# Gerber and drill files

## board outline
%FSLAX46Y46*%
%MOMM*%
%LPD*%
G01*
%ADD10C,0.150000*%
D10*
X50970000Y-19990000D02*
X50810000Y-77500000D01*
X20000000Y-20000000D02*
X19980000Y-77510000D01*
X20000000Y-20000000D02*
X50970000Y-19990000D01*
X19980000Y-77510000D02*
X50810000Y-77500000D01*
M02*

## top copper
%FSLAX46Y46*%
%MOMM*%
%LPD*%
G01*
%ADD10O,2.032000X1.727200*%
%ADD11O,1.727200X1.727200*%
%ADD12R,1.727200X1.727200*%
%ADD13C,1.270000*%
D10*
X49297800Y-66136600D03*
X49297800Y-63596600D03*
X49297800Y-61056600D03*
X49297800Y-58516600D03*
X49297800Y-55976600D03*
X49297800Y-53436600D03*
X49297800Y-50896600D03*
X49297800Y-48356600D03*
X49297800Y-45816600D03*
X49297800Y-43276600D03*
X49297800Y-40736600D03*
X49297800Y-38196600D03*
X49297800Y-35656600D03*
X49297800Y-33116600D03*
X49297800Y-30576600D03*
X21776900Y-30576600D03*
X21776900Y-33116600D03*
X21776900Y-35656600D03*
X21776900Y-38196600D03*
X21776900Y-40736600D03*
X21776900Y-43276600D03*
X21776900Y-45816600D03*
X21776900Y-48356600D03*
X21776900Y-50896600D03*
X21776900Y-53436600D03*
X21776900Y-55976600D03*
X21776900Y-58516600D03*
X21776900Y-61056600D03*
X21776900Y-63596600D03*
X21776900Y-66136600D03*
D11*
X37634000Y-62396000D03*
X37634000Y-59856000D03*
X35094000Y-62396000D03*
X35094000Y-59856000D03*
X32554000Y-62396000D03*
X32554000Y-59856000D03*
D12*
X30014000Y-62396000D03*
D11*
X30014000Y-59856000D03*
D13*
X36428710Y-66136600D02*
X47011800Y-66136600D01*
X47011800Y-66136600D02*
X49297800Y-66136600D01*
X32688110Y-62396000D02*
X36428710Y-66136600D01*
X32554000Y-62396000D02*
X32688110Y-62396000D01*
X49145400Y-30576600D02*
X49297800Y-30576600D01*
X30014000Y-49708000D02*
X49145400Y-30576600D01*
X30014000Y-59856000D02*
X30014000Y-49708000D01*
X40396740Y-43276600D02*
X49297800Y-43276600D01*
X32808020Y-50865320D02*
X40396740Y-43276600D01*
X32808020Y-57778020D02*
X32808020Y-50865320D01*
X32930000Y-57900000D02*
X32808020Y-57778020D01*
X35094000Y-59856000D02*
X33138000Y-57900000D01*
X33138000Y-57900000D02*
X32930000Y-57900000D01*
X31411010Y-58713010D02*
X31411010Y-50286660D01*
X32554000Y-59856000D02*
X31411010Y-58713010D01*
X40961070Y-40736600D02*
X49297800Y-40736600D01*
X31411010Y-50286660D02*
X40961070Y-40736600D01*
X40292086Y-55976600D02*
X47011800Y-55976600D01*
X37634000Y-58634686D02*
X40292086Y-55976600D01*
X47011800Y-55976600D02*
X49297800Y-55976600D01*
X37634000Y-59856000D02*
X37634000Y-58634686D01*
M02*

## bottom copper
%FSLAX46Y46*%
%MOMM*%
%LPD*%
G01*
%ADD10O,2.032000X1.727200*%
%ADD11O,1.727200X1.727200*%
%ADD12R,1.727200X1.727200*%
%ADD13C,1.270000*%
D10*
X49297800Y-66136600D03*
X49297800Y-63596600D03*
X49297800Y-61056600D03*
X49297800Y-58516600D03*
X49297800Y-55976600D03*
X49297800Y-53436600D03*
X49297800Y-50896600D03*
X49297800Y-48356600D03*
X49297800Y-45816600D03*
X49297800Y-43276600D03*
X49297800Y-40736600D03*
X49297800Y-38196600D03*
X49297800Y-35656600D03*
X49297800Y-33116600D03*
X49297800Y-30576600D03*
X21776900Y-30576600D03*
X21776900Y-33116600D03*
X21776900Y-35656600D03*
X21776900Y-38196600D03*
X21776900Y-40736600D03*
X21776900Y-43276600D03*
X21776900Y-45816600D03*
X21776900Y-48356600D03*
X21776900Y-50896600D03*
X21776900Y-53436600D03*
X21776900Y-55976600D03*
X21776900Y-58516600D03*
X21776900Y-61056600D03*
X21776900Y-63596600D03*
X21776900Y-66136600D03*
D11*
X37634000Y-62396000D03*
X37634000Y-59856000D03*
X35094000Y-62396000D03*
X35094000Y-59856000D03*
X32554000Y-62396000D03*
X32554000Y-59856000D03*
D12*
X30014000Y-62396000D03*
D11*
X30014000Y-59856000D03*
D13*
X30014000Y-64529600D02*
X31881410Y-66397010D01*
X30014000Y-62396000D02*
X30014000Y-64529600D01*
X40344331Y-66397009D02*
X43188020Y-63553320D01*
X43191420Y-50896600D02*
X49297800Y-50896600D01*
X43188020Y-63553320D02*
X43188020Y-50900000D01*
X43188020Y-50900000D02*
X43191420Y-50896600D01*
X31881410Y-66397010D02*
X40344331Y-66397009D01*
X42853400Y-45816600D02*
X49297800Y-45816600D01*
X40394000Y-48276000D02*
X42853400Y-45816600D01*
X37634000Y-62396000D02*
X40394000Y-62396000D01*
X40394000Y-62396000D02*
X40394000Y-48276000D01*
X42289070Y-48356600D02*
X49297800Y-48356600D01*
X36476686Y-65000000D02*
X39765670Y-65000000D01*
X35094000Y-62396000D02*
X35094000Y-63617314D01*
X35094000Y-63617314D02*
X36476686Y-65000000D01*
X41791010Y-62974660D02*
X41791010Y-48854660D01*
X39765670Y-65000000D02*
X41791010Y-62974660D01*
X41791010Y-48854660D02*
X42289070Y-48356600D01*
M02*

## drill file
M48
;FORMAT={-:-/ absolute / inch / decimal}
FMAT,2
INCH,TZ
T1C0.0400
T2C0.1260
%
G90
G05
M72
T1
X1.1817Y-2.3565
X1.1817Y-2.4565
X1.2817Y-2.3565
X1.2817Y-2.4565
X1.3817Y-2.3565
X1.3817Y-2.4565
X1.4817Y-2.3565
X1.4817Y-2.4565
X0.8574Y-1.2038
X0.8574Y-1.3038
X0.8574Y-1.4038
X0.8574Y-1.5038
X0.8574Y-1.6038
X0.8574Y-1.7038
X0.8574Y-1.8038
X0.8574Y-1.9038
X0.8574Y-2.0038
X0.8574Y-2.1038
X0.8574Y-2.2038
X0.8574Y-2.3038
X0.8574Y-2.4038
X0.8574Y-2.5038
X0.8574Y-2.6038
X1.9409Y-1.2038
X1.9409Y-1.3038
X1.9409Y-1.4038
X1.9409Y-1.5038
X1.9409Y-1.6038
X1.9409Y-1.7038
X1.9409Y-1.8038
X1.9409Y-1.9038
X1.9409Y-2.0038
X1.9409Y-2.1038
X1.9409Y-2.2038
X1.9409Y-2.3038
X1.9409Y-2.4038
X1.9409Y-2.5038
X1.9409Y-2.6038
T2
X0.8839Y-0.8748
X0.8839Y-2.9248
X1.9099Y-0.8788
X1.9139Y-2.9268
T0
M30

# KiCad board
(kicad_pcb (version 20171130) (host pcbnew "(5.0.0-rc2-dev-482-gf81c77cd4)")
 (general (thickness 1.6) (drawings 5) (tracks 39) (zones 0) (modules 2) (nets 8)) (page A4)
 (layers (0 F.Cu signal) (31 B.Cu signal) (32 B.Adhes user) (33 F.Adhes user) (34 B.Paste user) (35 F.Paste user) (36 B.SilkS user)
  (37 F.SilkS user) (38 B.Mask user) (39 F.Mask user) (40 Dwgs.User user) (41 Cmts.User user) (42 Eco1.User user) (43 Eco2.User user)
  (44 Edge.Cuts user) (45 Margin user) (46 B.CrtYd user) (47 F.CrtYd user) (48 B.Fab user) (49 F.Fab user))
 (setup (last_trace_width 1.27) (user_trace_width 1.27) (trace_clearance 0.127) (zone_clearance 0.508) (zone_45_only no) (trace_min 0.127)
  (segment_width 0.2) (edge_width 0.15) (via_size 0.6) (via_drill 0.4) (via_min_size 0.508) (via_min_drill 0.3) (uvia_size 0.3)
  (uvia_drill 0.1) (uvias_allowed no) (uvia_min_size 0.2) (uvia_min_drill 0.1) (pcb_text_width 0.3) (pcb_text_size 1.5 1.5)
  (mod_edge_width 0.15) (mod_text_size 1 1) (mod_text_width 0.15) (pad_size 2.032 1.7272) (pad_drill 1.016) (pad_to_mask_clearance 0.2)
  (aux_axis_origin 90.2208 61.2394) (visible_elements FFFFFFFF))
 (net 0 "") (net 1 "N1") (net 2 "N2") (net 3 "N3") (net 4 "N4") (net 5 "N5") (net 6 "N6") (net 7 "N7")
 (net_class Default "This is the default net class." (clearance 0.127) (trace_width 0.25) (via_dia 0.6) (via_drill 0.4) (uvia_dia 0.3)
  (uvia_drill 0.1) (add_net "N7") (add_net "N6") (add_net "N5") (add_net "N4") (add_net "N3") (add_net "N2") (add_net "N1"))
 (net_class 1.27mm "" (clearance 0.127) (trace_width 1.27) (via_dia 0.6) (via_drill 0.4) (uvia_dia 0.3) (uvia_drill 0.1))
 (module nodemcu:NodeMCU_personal (layer F.Cu) (at 20.5704 20.2896)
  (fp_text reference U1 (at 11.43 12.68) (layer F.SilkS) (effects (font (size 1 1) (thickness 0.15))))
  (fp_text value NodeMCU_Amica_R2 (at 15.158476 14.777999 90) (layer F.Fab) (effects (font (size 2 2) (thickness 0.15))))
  (pad "" np_thru_hole circle (at 27.94 2.032) (size 3.2 3.2) (drill 3.2) (layers *.Cu *.Mask))
  (pad 30 thru_hole oval (at 28.7274 45.847) (size 2.032 1.7272) (drill 1.016) (layers *.Cu *.Mask F.SilkS) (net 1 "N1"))
  (pad 29 thru_hole oval (at 28.7274 43.307) (size 2.032 1.7272) (drill 1.016) (layers *.Cu *.Mask F.SilkS))
  (pad 28 thru_hole oval (at 28.7274 40.767) (size 2.032 1.7272) (drill 1.016) (layers *.Cu *.Mask F.SilkS))
  (pad 27 thru_hole oval (at 28.7274 38.227) (size 2.032 1.7272) (drill 1.016) (layers *.Cu *.Mask F.SilkS))
  (pad 26 thru_hole oval (at 28.7274 35.687) (size 2.032 1.7272) (drill 1.016) (layers *.Cu *.Mask F.SilkS))
  (pad 25 thru_hole oval (at 28.7274 33.147) (size 2.032 1.7272) (drill 1.016) (layers *.Cu *.Mask F.SilkS))
  (pad 24 thru_hole oval (at 28.7274 30.607) (size 2.032 1.7272) (drill 1.016) (layers *.Cu *.Mask F.SilkS) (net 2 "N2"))
  (pad 23 thru_hole oval (at 28.7274 28.067) (size 2.032 1.7272) (drill 1.016) (layers *.Cu *.Mask F.SilkS) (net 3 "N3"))
  (pad 22 thru_hole oval (at 28.7274 25.527) (size 2.032 1.7272) (drill 1.016) (layers *.Cu *.Mask F.SilkS) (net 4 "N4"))
  (pad 21 thru_hole oval (at 28.7274 22.987) (size 2.032 1.7272) (drill 1.016) (layers *.Cu *.Mask F.SilkS) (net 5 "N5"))
  (pad 20 thru_hole oval (at 28.7274 20.447) (size 2.032 1.7272) (drill 1.016) (layers *.Cu *.Mask F.SilkS) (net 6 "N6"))
  (pad 19 thru_hole oval (at 28.7274 17.907) (size 2.032 1.7272) (drill 1.016) (layers *.Cu *.Mask F.SilkS))
  (pad 18 thru_hole oval (at 28.7274 15.367) (size 2.032 1.7272) (drill 1.016) (layers *.Cu *.Mask F.SilkS))
  (pad 17 thru_hole oval (at 28.7274 12.827) (size 2.032 1.7272) (drill 1.016) (layers *.Cu *.Mask F.SilkS))
  (pad 16 thru_hole oval (at 28.7274 10.287) (size 2.032 1.7272) (drill 1.016) (layers *.Cu *.Mask F.SilkS) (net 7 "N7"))
  (pad 1 thru_hole oval (at 1.2065 10.287) (size 2.032 1.7272) (drill 1.016) (layers *.Cu *.Mask F.SilkS))
  (pad 2 thru_hole oval (at 1.2065 12.827) (size 2.032 1.7272) (drill 1.016) (layers *.Cu *.Mask F.SilkS))
  (pad 3 thru_hole oval (at 1.2065 15.367) (size 2.032 1.7272) (drill 1.016) (layers *.Cu *.Mask F.SilkS))
  (pad 4 thru_hole oval (at 1.2065 17.907) (size 2.032 1.7272) (drill 1.016) (layers *.Cu *.Mask F.SilkS))
  (pad 5 thru_hole oval (at 1.2065 20.447) (size 2.032 1.7272) (drill 1.016) (layers *.Cu *.Mask F.SilkS))
  (pad 6 thru_hole oval (at 1.2065 22.987) (size 2.032 1.7272) (drill 1.016) (layers *.Cu *.Mask F.SilkS))
  (pad 7 thru_hole oval (at 1.2065 25.527) (size 2.032 1.7272) (drill 1.016) (layers *.Cu *.Mask F.SilkS))
  (pad 8 thru_hole oval (at 1.2065 28.067) (size 2.032 1.7272) (drill 1.016) (layers *.Cu *.Mask F.SilkS))
  (pad 9 thru_hole oval (at 1.2065 30.607) (size 2.032 1.7272) (drill 1.016) (layers *.Cu *.Mask F.SilkS))
  (pad 10 thru_hole oval (at 1.2065 33.147) (size 2.032 1.7272) (drill 1.016) (layers *.Cu *.Mask F.SilkS))
  (pad 11 thru_hole oval (at 1.2065 35.687) (size 2.032 1.7272) (drill 1.016) (layers *.Cu *.Mask F.SilkS))
  (pad 12 thru_hole oval (at 1.2065 38.227) (size 2.032 1.7272) (drill 1.016) (layers *.Cu *.Mask F.SilkS))
  (pad 13 thru_hole oval (at 1.2065 40.767) (size 2.032 1.7272) (drill 1.016) (layers *.Cu *.Mask F.SilkS))
  (pad 14 thru_hole oval (at 1.2065 43.307) (size 2.032 1.7272) (drill 1.016) (layers *.Cu *.Mask F.SilkS))
  (pad 15 thru_hole oval (at 1.2065 45.847) (size 2.032 1.7272) (drill 1.016) (layers *.Cu *.Mask F.SilkS))
  (pad "" np_thru_hole circle (at 1.8796 54.0004) (size 3.2 3.2) (drill 3.2) (layers *.Cu *.Mask))
  (pad "" np_thru_hole circle (at 28.0416 54.0512) (size 3.2 3.2) (drill 3.2) (layers *.Cu *.Mask))
  (pad "" np_thru_hole circle (at 1.8796 1.9304) (size 3.2 3.2) (drill 3.2) (layers *.Cu *.Mask)))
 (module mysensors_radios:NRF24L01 (layer F.Cu) (at 28.49 63.92 180)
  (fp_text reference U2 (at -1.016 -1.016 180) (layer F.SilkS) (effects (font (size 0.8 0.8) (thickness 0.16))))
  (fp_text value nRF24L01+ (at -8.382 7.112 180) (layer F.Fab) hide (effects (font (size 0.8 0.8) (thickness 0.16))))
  (pad 7 thru_hole oval (at -9.144 1.524 180) (size 1.7272 1.7272) (drill 1.016) (layers *.Cu *.Mask F.SilkS) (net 4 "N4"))
  (pad 8 thru_hole oval (at -9.144 4.064 180) (size 1.7272 1.7272) (drill 1.016) (layers *.Cu *.Mask F.SilkS))
  (pad 5 thru_hole oval (at -6.604 1.524 180) (size 1.7272 1.7272) (drill 1.016) (layers *.Cu *.Mask F.SilkS) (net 3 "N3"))
  (pad 6 thru_hole oval (at -6.604 4.064 180) (size 1.7272 1.7272) (drill 1.016) (layers *.Cu *.Mask F.SilkS) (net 5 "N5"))
  (pad 3 thru_hole oval (at -4.064 1.524 180) (size 1.7272 1.7272) (drill 1.016) (layers *.Cu *.Mask F.SilkS) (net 1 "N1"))
  (pad 4 thru_hole oval (at -4.064 4.064 180) (size 1.7272 1.7272) (drill 1.016) (layers *.Cu *.Mask F.SilkS) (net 6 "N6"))
  (pad 1 thru_hole rect (at -1.524 1.524 180) (size 1.7272 1.7272) (drill 1.016) (layers *.Cu *.Mask F.SilkS) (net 2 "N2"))
  (pad 2 thru_hole oval (at -1.524 4.064 180) (size 1.7272 1.7272) (drill 1.016) (layers *.Cu *.Mask F.SilkS) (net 7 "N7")))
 (gr_line (start 50.97 19.99) (end 50.81 77.5) (angle 90) (layer Edge.Cuts) (width 0.15))
 (gr_line (start 20 20) (end 19.98 77.51) (angle 90) (layer Edge.Cuts) (width 0.15))
 (gr_line (start 20 20) (end 50.97 19.99) (angle 90) (layer Edge.Cuts) (width 0.15))
 (gr_line (start 19.98 77.51) (end 50.81 77.5) (angle 90) (layer Edge.Cuts) (width 0.15))
 (segment (start 36.42871 66.1366) (end 47.0118 66.1366) (width 1.27) (layer F.Cu) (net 1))
 (segment (start 47.0118 66.1366) (end 49.2978 66.1366) (width 1.27) (layer F.Cu) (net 1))
 (segment (start 32.68811 62.396) (end 36.42871 66.1366) (width 1.27) (layer F.Cu) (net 1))
 (segment (start 32.554 62.396) (end 32.68811 62.396) (width 1.27) (layer F.Cu) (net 1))
 (segment (start 49.1454 30.5766) (end 49.2978 30.5766) (width 1.27) (layer F.Cu) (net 7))
 (segment (start 30.014 49.708) (end 49.1454 30.5766) (width 1.27) (layer F.Cu) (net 7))
 (segment (start 30.014 59.856) (end 30.014 49.708) (width 1.27) (layer F.Cu) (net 7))
 (segment (start 40.39674 43.2766) (end 49.2978 43.2766) (width 1.27) (layer F.Cu) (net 5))
 (segment (start 32.80802 50.86532) (end 40.39674 43.2766) (width 1.27) (layer F.Cu) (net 5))
 (segment (start 32.80802 57.77802) (end 32.80802 50.86532) (width 1.27) (layer F.Cu) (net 5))
 (segment (start 32.93 57.9) (end 32.80802 57.77802) (width 1.27) (layer F.Cu) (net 5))
 (segment (start 35.094 59.856) (end 33.138 57.9) (width 1.27) (layer F.Cu) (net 5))
 (segment (start 33.138 57.9) (end 32.93 57.9) (width 1.27) (layer F.Cu) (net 5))
 (segment (start 31.41101 58.71301) (end 31.41101 50.28666) (width 1.27) (layer F.Cu) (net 6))
 (segment (start 32.554 59.856) (end 31.41101 58.71301) (width 1.27) (layer F.Cu) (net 6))
 (segment (start 40.96107 40.7366) (end 49.2978 40.7366) (width 1.27) (layer F.Cu) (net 6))
 (segment (start 31.41101 50.28666) (end 40.96107 40.7366) (width 1.27) (layer F.Cu) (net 6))
 (segment (start 40.292086 55.9766) (end 47.0118 55.9766) (width 1.27) (layer F.Cu) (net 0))
 (segment (start 37.634 58.634686) (end 40.292086 55.9766) (width 1.27) (layer F.Cu) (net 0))
 (segment (start 47.0118 55.9766) (end 49.2978 55.9766) (width 1.27) (layer F.Cu) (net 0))
 (segment (start 37.634 59.856) (end 37.634 58.634686) (width 1.27) (layer F.Cu) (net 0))
 (segment (start 30.014 64.5296) (end 31.88141 66.39701) (width 1.27) (layer B.Cu) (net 2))
 (segment (start 30.014 62.396) (end 30.014 64.5296) (width 1.27) (layer B.Cu) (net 2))
 (segment (start 40.344331 66.397009) (end 43.18802 63.55332) (width 1.27) (layer B.Cu) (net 2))
 (segment (start 43.19142 50.8966) (end 49.2978 50.8966) (width 1.27) (layer B.Cu) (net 2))
 (segment (start 43.18802 63.55332) (end 43.18802 50.9) (width 1.27) (layer B.Cu) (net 2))
 (segment (start 43.18802 50.9) (end 43.19142 50.8966) (width 1.27) (layer B.Cu) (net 2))
 (segment (start 31.88141 66.39701) (end 40.344331 66.397009) (width 1.27) (layer B.Cu) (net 2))
 (segment (start 42.8534 45.8166) (end 49.2978 45.8166) (width 1.27) (layer B.Cu) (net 4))
 (segment (start 40.394 48.276) (end 42.8534 45.8166) (width 1.27) (layer B.Cu) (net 4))
 (segment (start 37.634 62.396) (end 40.394 62.396) (width 1.27) (layer B.Cu) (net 4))
 (segment (start 40.394 62.396) (end 40.394 48.276) (width 1.27) (layer B.Cu) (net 4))
 (segment (start 42.28907 48.3566) (end 49.2978 48.3566) (width 1.27) (layer B.Cu) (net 3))
 (segment (start 36.476686 65) (end 39.76567 65) (width 1.27) (layer B.Cu) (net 3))
 (segment (start 35.094 62.396) (end 35.094 63.617314) (width 1.27) (layer B.Cu) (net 3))
 (segment (start 35.094 63.617314) (end 36.476686 65) (width 1.27) (layer B.Cu) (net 3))
 (segment (start 41.79101 62.97466) (end 41.79101 48.85466) (width 1.27) (layer B.Cu) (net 3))
 (segment (start 39.76567 65) (end 41.79101 62.97466) (width 1.27) (layer B.Cu) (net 3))
 (segment (start 41.79101 48.85466) (end 42.28907 48.3566) (width 1.27) (layer B.Cu) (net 3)))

